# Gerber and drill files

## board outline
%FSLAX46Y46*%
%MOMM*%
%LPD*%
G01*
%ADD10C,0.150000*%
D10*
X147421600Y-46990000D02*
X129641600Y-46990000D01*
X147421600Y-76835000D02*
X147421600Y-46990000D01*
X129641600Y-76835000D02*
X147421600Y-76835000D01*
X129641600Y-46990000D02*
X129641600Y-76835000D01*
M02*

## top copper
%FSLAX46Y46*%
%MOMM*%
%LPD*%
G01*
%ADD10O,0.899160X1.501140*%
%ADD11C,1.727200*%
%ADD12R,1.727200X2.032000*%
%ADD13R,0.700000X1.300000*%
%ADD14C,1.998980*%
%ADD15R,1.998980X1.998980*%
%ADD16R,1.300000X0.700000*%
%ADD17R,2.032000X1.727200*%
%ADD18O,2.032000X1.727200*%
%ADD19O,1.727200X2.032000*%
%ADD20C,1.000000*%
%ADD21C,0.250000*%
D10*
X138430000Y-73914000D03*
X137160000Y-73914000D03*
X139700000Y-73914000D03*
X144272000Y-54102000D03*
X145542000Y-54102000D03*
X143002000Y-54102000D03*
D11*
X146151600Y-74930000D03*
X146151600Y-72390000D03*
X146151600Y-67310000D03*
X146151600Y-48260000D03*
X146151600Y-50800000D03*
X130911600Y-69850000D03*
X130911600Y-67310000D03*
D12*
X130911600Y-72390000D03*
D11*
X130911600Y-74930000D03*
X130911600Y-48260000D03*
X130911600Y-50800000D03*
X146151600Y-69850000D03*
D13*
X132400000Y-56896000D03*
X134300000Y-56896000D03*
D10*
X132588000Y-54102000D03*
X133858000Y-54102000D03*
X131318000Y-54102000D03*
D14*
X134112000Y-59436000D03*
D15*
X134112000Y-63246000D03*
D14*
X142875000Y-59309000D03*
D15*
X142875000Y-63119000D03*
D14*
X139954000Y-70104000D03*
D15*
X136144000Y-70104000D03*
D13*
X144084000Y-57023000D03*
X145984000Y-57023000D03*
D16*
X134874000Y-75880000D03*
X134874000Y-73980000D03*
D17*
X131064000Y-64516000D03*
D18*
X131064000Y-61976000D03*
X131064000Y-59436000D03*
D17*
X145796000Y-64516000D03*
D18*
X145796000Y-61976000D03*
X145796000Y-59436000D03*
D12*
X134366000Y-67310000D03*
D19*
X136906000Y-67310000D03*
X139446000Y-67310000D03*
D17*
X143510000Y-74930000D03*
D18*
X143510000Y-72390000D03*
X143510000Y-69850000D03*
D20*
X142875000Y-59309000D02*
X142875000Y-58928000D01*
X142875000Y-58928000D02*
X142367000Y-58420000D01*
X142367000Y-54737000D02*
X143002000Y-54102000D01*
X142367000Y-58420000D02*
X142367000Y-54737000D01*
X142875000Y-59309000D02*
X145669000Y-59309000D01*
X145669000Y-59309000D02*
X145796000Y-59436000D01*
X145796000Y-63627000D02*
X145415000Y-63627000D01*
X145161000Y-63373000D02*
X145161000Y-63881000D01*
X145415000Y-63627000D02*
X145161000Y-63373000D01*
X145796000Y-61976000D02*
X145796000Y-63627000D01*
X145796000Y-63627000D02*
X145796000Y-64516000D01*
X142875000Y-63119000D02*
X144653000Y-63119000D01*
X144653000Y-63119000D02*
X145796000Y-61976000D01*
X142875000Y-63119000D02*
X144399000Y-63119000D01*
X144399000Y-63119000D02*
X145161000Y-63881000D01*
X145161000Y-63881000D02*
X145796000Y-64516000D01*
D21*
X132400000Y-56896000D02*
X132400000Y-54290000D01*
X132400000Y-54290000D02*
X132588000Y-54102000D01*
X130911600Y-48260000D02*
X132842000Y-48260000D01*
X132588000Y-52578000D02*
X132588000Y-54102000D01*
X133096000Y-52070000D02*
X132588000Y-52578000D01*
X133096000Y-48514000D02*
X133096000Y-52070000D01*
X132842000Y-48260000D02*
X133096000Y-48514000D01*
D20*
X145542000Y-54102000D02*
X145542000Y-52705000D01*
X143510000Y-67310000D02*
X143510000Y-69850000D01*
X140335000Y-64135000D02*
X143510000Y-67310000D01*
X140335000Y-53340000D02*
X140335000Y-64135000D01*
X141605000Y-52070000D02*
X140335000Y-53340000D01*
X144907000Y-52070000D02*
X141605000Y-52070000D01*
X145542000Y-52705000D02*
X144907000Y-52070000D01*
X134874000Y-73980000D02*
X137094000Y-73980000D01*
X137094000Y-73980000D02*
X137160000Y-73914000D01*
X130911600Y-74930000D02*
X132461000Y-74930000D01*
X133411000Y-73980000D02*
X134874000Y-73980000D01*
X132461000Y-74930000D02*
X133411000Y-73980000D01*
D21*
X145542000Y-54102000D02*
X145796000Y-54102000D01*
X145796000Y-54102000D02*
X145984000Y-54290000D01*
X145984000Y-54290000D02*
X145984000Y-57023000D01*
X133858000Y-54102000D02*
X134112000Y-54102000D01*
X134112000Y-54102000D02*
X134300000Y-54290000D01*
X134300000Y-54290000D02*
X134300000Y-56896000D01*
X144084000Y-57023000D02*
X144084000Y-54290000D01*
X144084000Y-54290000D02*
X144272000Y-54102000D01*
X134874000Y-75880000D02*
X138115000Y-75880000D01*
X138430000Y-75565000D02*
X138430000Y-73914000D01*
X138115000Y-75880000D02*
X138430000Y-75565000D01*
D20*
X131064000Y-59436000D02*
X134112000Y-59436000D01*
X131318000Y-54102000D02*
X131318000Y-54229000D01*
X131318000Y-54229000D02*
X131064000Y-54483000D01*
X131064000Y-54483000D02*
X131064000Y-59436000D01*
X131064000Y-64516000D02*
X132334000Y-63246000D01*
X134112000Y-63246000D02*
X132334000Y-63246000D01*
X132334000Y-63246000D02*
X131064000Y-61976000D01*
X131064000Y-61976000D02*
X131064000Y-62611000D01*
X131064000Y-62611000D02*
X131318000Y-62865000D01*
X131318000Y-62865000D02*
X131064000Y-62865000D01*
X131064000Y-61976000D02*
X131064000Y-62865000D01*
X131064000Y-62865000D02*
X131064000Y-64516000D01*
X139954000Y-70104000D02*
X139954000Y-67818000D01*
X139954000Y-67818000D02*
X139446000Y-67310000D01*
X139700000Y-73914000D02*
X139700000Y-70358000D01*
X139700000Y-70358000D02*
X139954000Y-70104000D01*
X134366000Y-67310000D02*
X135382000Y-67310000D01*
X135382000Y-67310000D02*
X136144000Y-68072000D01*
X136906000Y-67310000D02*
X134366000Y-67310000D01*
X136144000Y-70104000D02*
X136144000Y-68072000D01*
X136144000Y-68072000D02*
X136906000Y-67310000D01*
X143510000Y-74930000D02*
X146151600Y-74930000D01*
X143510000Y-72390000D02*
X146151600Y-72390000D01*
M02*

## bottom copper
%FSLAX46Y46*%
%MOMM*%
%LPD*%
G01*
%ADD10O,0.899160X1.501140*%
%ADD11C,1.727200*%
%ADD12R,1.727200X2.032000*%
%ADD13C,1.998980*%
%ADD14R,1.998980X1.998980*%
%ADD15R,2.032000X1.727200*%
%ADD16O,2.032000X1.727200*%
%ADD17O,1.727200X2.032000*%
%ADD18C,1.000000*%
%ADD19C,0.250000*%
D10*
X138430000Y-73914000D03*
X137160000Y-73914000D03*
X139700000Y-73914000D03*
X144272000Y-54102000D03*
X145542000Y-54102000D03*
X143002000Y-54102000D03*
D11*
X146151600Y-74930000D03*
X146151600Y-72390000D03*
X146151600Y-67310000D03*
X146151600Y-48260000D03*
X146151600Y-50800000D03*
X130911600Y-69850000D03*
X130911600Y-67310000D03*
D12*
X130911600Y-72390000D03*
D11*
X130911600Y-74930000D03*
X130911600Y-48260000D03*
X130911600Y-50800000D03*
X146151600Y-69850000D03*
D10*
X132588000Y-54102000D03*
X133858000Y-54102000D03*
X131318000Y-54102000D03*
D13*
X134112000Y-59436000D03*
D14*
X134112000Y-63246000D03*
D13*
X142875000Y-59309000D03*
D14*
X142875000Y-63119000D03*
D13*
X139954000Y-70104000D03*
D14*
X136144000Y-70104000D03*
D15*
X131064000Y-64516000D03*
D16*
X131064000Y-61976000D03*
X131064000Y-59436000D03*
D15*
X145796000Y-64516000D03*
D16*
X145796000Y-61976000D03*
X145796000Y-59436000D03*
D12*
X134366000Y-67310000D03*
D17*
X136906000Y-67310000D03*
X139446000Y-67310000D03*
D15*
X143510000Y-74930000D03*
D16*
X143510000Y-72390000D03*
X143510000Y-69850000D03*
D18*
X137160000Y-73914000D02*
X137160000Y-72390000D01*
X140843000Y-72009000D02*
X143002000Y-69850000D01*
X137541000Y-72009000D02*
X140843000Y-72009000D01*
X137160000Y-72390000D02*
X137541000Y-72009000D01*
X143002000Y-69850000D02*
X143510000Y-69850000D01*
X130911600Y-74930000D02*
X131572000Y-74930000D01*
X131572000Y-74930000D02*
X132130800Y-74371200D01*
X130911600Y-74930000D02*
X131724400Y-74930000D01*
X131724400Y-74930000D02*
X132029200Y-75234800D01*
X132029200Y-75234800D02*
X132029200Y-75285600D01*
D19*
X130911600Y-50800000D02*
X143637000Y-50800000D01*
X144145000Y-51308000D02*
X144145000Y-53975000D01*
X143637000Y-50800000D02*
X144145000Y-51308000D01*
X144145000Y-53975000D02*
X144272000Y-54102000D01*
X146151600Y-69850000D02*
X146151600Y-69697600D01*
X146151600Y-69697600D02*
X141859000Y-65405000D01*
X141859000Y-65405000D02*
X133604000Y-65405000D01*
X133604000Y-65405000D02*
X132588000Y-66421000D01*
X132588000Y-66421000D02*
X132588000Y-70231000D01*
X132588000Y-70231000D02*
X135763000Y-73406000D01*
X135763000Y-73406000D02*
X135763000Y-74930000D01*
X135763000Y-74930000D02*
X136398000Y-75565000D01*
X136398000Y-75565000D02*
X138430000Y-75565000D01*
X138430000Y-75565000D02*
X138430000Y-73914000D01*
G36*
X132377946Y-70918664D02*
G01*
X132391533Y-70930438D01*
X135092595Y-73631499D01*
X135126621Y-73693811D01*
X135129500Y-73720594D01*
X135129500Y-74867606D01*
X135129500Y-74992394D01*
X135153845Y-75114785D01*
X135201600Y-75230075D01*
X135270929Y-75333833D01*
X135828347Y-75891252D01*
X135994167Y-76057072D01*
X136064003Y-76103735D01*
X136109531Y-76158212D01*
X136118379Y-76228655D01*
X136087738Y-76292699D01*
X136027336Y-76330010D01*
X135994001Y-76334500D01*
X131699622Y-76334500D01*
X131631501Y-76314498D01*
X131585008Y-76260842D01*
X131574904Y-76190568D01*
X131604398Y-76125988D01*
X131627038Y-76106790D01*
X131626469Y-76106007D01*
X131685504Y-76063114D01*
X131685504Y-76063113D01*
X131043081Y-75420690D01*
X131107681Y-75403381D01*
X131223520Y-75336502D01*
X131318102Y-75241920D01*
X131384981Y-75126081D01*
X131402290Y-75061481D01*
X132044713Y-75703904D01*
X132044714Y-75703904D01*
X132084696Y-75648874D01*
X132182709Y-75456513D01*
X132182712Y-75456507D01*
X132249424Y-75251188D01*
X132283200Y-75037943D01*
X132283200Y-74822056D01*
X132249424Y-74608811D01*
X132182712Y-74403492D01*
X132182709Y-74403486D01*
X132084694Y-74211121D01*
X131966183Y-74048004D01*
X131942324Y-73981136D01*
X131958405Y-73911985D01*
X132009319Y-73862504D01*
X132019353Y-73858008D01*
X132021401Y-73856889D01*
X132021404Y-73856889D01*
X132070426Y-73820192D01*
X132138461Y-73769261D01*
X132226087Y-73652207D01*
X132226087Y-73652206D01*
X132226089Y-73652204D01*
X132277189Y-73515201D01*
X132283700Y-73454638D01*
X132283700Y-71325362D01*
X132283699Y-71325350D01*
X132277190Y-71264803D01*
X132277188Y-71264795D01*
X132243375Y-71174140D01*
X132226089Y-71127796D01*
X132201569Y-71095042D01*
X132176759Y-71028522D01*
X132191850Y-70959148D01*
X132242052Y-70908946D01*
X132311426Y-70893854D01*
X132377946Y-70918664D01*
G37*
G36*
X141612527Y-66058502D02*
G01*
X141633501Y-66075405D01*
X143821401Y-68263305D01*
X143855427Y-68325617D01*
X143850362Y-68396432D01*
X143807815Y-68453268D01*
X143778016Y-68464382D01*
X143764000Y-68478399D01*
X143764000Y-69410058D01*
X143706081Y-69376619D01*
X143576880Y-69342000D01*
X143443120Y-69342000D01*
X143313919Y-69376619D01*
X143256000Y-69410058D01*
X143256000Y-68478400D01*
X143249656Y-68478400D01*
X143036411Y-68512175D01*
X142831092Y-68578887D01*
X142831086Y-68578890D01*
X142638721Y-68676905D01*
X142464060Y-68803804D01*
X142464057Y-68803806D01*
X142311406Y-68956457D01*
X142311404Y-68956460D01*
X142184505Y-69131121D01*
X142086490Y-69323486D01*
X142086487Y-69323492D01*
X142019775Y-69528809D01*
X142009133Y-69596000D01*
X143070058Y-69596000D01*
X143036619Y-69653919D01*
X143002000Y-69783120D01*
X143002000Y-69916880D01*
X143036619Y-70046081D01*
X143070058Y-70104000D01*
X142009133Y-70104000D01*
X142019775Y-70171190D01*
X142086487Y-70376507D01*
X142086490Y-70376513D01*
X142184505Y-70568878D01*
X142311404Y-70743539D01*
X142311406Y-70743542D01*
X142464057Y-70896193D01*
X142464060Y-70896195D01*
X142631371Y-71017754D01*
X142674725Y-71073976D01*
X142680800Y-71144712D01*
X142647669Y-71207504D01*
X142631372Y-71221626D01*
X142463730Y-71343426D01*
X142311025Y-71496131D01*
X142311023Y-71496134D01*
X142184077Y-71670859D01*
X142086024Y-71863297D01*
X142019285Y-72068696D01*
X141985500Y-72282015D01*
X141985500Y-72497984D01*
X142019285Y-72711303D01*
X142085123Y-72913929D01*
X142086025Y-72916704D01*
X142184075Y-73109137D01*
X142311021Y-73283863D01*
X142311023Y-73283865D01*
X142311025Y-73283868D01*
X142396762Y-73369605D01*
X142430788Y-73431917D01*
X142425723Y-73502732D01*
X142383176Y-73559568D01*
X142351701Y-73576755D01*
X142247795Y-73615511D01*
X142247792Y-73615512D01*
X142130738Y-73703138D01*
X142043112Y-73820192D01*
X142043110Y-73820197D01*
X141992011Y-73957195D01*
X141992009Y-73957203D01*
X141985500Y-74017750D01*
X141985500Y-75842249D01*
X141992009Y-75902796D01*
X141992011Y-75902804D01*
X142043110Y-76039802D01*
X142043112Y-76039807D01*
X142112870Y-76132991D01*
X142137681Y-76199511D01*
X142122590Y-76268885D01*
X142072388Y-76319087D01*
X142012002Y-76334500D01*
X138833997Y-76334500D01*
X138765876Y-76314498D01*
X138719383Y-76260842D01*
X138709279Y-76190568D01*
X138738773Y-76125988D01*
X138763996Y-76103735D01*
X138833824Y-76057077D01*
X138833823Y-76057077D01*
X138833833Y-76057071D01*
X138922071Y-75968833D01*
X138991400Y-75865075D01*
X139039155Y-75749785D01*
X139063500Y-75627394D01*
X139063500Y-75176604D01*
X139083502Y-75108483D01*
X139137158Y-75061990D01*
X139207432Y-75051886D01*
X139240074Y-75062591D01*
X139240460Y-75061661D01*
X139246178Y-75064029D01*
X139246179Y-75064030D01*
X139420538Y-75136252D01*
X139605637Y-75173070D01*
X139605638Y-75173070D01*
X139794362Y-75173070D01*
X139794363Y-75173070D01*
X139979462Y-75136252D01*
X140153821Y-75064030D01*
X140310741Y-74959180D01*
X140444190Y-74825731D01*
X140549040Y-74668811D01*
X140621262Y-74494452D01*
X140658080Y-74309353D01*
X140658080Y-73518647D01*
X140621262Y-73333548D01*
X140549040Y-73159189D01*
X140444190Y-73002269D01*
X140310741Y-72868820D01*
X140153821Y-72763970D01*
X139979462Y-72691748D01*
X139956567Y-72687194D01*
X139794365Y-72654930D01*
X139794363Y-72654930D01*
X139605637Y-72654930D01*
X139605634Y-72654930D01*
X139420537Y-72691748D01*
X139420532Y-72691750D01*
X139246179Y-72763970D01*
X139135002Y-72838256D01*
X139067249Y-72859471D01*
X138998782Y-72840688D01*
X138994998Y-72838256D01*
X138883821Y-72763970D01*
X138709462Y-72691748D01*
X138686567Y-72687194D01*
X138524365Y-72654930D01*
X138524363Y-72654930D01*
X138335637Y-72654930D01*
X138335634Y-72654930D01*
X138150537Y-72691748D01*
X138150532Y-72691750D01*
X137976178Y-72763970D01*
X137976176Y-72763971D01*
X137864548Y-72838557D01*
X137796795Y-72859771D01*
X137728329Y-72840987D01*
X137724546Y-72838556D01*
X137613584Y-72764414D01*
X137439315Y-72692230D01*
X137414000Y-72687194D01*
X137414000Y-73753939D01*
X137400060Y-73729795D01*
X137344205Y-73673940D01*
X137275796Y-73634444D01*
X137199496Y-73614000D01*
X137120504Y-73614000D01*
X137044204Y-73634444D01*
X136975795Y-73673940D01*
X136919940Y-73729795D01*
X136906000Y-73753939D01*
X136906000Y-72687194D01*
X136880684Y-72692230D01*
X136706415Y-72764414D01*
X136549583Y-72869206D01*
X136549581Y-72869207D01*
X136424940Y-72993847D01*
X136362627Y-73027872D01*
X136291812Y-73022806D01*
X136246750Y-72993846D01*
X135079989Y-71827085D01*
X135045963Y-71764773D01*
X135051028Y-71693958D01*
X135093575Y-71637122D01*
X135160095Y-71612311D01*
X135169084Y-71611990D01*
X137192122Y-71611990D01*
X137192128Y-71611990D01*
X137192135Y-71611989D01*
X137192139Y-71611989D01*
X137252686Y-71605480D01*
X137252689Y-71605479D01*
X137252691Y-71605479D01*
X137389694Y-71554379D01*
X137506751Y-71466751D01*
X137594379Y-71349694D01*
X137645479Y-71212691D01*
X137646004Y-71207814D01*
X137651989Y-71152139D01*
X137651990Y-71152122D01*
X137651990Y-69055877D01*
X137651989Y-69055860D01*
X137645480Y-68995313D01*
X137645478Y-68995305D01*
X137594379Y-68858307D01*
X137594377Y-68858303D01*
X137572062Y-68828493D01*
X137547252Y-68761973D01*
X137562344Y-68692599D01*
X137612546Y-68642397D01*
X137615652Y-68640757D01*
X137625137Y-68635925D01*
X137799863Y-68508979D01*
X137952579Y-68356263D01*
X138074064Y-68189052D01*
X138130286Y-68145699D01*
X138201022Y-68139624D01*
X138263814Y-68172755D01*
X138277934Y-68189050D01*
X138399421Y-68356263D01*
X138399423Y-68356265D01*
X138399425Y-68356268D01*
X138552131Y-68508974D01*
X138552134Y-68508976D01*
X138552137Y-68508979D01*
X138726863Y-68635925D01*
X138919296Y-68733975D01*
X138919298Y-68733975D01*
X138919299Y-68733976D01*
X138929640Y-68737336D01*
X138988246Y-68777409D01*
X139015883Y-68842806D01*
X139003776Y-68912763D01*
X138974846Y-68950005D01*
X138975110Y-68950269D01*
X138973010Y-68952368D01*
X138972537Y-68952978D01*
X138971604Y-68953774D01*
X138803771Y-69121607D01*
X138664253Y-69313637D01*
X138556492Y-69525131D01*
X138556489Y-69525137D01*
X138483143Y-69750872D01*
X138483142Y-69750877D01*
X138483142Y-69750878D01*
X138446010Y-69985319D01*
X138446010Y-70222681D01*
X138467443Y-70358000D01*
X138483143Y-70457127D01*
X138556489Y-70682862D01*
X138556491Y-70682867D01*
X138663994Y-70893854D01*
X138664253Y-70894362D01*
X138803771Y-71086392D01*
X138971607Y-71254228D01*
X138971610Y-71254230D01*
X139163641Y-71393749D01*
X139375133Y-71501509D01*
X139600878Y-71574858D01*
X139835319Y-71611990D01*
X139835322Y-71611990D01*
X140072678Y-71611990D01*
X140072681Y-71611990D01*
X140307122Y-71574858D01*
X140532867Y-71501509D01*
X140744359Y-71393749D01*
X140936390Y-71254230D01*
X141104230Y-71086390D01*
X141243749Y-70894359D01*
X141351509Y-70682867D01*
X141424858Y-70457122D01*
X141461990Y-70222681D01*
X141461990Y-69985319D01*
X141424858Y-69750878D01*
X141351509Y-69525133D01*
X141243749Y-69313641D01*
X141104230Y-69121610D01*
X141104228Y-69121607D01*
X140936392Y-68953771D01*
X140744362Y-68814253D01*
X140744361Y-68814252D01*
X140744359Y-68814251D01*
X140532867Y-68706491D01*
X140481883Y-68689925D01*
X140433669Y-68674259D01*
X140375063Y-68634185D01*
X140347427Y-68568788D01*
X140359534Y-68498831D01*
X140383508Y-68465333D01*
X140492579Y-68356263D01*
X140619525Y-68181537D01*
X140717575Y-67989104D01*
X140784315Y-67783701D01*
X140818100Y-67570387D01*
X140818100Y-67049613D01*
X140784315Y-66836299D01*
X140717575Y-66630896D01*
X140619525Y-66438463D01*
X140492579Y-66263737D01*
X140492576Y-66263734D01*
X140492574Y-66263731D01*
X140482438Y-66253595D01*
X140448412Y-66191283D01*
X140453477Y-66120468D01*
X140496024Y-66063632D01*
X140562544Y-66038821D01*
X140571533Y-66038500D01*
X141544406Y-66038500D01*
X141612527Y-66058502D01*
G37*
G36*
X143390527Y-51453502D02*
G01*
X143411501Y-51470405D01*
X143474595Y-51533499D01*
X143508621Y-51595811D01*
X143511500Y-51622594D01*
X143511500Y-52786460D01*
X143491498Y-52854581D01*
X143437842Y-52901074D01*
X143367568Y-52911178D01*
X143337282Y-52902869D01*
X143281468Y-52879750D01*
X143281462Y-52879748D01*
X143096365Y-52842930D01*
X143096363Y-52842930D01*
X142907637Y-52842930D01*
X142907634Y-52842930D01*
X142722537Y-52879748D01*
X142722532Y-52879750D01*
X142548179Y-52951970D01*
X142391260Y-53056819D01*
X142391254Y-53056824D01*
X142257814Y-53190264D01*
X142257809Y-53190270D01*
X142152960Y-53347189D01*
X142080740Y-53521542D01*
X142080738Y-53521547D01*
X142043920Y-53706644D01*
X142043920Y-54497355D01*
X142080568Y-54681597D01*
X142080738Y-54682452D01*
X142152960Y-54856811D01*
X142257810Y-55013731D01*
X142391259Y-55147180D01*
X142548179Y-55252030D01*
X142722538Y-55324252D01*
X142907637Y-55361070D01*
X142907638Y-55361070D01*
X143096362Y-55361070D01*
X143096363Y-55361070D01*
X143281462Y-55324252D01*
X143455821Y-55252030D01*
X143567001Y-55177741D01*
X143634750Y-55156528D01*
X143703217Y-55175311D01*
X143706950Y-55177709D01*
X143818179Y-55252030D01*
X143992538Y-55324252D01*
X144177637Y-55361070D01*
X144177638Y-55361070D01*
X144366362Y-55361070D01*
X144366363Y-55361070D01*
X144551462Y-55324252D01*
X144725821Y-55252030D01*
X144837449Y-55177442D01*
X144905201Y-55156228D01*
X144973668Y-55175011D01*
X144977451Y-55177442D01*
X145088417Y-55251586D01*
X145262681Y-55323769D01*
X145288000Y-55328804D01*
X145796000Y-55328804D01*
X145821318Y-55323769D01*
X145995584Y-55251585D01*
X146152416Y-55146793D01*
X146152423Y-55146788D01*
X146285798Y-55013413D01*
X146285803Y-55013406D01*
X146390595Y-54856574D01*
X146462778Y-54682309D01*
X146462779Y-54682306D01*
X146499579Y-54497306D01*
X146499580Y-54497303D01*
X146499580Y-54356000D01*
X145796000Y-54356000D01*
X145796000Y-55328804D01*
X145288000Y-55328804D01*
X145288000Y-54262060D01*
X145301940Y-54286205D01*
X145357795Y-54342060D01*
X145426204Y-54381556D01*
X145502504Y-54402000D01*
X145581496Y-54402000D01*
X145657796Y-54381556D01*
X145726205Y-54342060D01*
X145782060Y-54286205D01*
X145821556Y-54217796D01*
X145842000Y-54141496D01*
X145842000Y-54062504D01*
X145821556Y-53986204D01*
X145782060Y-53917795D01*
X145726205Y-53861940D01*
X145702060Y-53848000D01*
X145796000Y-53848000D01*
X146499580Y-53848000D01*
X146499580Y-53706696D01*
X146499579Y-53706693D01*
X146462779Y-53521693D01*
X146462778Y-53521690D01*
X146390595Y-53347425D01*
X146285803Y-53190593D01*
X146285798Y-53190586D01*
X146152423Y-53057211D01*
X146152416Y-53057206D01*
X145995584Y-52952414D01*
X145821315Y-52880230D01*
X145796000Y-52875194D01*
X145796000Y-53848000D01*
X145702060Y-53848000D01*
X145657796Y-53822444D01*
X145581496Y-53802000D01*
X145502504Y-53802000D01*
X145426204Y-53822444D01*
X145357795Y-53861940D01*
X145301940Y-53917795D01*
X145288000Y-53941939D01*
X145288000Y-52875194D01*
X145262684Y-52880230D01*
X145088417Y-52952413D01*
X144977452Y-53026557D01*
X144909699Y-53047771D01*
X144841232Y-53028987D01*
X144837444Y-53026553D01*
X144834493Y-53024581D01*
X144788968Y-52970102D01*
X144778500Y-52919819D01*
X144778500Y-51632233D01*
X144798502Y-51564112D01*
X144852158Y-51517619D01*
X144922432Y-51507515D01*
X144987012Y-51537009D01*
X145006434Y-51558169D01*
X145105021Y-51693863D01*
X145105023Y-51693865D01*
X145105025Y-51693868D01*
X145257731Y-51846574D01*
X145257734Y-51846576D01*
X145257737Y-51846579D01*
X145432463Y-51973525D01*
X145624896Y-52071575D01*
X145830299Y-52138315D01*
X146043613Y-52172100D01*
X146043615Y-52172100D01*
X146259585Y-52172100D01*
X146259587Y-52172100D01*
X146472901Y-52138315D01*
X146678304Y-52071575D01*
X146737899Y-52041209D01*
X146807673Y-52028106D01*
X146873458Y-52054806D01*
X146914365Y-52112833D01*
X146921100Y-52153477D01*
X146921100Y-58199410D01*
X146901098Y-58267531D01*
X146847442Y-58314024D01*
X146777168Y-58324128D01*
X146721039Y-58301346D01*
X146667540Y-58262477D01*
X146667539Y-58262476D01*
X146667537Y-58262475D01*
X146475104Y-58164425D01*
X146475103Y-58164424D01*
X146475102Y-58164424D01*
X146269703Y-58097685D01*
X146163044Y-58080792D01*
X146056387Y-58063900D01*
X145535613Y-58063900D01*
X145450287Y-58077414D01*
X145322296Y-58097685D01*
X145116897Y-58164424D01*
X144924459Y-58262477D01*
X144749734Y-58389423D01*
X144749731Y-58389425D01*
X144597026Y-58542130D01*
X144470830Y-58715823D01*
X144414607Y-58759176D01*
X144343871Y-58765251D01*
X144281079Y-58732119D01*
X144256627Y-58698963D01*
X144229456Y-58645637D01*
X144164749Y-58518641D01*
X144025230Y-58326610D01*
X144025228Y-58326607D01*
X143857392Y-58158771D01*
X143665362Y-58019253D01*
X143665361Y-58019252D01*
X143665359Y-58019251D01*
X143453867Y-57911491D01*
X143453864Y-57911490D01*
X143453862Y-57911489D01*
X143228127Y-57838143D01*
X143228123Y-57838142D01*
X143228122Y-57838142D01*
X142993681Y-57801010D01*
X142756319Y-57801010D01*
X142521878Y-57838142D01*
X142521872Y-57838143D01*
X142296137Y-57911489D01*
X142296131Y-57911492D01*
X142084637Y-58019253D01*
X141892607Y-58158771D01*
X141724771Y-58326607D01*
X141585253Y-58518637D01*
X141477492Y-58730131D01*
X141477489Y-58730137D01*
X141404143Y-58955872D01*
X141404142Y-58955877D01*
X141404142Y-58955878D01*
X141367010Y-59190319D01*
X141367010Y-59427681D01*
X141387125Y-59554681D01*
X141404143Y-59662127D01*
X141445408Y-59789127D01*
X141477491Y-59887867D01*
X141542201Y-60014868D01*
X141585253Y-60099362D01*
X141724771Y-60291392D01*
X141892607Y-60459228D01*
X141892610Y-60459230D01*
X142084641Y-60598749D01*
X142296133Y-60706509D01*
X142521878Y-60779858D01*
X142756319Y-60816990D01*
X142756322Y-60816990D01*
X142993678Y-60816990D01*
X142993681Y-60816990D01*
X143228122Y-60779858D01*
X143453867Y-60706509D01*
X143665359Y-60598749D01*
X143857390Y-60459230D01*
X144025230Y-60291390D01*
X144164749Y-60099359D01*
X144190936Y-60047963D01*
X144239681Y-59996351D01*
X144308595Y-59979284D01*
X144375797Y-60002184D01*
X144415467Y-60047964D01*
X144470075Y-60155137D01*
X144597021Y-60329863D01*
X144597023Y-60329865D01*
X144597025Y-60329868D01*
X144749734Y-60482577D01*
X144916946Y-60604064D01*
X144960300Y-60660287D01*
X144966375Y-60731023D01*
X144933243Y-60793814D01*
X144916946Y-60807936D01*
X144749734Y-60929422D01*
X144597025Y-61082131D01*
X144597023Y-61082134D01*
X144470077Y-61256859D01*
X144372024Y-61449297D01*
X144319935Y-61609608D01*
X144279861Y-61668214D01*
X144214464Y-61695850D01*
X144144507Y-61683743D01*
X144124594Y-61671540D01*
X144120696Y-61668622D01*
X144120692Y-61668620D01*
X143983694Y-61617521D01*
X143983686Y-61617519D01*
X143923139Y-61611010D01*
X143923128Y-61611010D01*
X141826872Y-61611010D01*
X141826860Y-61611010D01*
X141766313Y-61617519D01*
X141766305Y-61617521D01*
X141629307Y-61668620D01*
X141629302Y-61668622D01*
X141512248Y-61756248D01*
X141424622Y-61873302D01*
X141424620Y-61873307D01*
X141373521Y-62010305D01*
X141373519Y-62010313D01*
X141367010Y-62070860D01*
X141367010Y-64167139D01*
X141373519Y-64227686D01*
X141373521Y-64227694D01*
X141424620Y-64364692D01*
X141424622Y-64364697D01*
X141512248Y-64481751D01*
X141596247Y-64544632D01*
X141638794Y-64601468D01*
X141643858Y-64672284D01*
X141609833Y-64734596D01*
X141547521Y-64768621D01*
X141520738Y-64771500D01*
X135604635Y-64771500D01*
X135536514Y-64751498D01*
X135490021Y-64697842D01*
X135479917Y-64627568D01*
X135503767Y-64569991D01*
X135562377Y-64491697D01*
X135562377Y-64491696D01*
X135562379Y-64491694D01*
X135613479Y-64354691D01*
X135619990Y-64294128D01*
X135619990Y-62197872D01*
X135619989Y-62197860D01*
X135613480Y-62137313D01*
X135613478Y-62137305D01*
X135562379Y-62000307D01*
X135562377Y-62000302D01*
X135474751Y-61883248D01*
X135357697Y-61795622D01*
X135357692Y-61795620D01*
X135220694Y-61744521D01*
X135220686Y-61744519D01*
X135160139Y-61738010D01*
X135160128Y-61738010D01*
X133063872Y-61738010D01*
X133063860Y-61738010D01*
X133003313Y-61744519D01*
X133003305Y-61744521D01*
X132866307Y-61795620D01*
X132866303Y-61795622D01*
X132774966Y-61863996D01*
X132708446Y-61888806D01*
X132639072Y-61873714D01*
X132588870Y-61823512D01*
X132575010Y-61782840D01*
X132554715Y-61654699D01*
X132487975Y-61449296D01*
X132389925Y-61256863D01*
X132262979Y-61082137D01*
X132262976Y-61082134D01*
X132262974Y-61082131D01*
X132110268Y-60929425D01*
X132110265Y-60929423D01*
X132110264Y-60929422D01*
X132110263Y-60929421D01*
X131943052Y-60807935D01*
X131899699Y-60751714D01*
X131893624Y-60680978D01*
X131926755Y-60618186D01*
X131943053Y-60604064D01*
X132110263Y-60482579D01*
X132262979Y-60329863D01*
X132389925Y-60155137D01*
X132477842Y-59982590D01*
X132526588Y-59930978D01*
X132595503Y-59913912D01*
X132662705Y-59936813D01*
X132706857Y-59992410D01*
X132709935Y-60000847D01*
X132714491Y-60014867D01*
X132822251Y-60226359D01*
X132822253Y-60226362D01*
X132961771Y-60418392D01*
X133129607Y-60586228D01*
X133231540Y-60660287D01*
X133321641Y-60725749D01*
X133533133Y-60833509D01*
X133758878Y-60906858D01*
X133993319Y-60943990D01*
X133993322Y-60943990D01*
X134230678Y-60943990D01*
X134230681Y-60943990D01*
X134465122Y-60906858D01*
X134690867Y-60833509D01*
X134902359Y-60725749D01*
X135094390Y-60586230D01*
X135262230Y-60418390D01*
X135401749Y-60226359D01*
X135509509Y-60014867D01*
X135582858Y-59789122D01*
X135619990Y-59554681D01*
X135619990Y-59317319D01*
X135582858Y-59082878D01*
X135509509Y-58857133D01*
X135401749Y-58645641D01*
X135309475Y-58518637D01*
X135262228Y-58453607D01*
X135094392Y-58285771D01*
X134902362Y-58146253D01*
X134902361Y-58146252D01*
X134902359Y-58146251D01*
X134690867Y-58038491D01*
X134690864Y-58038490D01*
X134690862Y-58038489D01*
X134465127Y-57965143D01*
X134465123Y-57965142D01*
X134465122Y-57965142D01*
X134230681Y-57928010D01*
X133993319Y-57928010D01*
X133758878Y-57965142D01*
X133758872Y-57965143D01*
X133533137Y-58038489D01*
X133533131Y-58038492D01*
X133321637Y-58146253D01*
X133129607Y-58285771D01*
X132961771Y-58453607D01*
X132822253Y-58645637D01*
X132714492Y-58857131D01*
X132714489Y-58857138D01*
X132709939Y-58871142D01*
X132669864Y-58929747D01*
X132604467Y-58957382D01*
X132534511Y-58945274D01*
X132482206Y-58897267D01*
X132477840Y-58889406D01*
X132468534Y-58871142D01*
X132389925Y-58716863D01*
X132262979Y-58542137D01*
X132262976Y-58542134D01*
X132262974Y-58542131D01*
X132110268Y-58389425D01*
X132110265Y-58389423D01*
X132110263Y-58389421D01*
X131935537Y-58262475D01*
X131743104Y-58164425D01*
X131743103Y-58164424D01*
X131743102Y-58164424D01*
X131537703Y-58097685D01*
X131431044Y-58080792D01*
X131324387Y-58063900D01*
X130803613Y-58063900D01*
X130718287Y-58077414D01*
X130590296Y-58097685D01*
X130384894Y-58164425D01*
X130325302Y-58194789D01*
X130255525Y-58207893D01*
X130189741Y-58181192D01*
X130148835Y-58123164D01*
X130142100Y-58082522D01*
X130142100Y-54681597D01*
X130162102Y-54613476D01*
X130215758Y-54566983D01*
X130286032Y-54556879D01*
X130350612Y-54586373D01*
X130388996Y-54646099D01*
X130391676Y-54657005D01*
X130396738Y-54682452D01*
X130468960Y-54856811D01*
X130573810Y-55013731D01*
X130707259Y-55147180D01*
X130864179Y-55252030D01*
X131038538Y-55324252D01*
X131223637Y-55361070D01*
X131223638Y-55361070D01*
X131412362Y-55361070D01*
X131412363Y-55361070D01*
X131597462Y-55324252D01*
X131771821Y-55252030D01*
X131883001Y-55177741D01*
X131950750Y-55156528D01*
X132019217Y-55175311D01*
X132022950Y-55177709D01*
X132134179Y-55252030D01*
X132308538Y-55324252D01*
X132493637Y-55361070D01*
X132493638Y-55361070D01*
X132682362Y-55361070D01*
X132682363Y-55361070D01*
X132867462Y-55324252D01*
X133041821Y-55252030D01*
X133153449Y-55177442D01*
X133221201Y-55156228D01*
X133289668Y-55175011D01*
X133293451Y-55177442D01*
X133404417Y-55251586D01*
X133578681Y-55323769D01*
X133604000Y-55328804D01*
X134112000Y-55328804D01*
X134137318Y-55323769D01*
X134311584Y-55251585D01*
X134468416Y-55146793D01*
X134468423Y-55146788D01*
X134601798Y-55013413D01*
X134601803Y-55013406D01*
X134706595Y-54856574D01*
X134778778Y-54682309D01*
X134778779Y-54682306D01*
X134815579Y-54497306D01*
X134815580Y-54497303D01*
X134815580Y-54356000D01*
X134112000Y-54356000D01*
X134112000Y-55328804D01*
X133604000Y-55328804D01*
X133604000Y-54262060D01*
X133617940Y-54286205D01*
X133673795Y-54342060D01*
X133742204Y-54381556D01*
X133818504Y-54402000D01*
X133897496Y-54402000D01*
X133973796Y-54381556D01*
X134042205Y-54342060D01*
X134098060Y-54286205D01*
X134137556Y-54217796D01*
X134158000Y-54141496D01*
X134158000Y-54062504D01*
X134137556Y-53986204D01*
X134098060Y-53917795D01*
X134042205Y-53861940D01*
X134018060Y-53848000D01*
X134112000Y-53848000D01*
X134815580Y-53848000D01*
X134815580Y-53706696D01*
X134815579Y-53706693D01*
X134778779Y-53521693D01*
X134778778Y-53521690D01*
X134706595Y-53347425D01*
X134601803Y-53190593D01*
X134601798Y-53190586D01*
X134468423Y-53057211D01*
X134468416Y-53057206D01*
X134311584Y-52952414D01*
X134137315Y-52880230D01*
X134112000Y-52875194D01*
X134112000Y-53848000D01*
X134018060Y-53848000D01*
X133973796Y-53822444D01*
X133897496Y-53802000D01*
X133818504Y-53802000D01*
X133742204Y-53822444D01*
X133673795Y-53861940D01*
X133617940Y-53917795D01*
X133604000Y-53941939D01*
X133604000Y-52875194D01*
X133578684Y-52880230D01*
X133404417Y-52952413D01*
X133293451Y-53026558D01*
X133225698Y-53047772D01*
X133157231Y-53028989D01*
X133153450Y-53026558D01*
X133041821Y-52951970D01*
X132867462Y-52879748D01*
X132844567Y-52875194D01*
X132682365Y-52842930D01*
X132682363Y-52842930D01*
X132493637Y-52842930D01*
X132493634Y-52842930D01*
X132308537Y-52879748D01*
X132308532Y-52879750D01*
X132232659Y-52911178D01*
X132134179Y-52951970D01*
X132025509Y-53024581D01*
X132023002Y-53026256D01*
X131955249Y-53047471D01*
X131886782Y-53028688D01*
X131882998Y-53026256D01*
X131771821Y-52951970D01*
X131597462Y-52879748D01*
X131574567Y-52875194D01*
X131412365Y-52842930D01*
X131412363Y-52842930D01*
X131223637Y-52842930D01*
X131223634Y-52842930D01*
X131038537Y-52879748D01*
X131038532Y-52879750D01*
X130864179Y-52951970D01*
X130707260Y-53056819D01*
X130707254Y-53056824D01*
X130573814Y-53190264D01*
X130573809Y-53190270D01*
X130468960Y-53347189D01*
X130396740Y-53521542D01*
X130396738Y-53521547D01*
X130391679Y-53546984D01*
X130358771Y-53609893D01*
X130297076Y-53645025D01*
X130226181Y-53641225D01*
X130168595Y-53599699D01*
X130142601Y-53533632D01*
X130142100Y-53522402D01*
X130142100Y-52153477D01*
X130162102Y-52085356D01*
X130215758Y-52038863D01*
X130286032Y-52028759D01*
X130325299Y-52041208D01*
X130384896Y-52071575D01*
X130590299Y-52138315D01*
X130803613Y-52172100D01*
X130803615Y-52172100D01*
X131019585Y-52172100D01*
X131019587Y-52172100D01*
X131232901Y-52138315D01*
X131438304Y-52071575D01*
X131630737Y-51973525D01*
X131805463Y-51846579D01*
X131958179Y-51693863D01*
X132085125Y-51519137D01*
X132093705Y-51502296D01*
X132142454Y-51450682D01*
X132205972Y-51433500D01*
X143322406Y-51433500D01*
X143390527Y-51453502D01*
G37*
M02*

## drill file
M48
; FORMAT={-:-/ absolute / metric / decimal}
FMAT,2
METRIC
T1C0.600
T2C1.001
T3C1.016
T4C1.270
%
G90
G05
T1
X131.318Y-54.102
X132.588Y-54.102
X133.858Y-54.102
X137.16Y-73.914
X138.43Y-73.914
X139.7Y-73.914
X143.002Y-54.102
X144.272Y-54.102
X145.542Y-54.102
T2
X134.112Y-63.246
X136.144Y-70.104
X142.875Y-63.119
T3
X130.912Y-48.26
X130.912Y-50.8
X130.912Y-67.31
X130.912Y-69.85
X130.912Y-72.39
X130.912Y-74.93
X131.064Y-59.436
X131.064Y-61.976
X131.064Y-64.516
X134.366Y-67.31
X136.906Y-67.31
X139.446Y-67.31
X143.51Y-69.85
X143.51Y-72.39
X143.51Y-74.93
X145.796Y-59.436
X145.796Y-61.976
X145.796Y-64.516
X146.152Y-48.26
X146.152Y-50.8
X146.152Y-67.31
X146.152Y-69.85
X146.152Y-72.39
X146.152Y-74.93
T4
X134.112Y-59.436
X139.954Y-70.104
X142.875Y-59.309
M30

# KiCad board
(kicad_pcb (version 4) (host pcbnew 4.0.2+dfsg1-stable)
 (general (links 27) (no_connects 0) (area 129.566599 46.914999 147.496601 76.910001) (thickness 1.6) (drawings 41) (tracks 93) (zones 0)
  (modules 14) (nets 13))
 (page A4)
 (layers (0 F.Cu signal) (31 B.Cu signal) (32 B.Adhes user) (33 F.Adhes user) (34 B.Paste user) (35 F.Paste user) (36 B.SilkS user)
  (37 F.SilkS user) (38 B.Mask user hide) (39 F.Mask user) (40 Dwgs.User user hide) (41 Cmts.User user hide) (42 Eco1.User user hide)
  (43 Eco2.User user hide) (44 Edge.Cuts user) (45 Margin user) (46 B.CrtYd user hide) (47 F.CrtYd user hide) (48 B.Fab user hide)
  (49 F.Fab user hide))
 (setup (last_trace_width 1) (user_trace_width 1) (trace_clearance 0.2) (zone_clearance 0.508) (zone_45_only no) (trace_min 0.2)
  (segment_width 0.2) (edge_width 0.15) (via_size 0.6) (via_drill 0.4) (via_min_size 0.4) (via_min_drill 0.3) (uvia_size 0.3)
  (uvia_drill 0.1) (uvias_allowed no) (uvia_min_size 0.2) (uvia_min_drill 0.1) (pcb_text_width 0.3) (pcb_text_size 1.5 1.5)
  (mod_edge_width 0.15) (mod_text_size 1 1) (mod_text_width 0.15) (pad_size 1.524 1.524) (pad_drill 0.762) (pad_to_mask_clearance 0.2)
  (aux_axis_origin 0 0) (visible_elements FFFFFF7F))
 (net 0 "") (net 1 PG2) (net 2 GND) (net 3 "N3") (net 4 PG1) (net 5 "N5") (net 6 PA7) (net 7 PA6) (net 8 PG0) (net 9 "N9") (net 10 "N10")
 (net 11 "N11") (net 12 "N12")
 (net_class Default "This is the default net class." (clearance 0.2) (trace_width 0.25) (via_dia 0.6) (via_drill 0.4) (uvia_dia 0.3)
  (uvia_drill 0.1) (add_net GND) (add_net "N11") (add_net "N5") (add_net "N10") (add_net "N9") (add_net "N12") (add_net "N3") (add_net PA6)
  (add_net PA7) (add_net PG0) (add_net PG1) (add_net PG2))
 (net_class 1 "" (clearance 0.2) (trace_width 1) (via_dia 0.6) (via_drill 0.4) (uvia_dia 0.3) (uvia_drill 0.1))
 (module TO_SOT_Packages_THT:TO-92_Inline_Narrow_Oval (layer F.Cu) (at 139.7 73.914 180)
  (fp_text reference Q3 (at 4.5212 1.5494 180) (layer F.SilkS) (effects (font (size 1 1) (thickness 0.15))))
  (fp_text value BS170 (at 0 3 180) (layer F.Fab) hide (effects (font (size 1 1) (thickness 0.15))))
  (pad 2 thru_hole oval (at 1.27 0) (size 0.89916 1.50114) (drill 0.6) (layers *.Cu *.Mask F.SilkS) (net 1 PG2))
  (pad 3 thru_hole oval (at 2.54 0) (size 0.89916 1.50114) (drill 0.6) (layers *.Cu *.Mask F.SilkS) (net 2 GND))
  (pad 1 thru_hole oval (at 0 0) (size 0.89916 1.50114) (drill 0.6) (layers *.Cu *.Mask F.SilkS) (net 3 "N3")))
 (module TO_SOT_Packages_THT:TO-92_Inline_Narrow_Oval (layer F.Cu) (at 143.002 54.102)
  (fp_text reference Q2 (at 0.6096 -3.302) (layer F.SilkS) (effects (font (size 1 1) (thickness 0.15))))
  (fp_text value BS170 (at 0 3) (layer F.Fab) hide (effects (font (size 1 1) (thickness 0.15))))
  (pad 2 thru_hole oval (at 1.27 0 180) (size 0.89916 1.50114) (drill 0.6) (layers *.Cu *.Mask F.SilkS) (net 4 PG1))
  (pad 3 thru_hole oval (at 2.54 0 180) (size 0.89916 1.50114) (drill 0.6) (layers *.Cu *.Mask F.SilkS) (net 2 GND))
  (pad 1 thru_hole oval (at 0 0 180) (size 0.89916 1.50114) (drill 0.6) (layers *.Cu *.Mask F.SilkS) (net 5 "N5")))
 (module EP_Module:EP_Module (layer F.Cu) (at 133.4516 48.26)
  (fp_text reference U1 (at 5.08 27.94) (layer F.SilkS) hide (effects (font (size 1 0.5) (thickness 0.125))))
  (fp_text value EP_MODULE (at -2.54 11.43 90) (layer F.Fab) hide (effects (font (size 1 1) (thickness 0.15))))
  (pad 12 thru_hole circle (at 12.7 26.67) (size 1.7272 1.7272) (drill 1.016) (layers *.Cu *.Mask F.SilkS) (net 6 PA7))
  (pad 11 thru_hole circle (at 12.7 24.13) (size 1.7272 1.7272) (drill 1.016) (layers *.Cu *.Mask F.SilkS) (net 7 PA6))
  (pad 10 thru_hole circle (at 12.7 19.05) (size 1.7272 1.7272) (drill 1.016) (layers *.Cu *.Mask F.SilkS))
  (pad 9 thru_hole circle (at 12.7 0) (size 1.7272 1.7272) (drill 1.016) (layers *.Cu *.Mask F.SilkS))
  (pad 8 thru_hole circle (at 12.7 2.54) (size 1.7272 1.7272) (drill 1.016) (layers *.Cu *.Mask F.SilkS))
  (pad 7 thru_hole circle (at -2.54 21.59) (size 1.7272 1.7272) (drill 1.016) (layers *.Cu *.Mask F.SilkS))
  (pad 6 thru_hole circle (at -2.54 19.05) (size 1.7272 1.7272) (drill 1.016) (layers *.Cu *.Mask F.SilkS))
  (pad 1 thru_hole rect (at -2.54 24.13) (size 1.7272 2.032) (drill 1.016) (layers *.Cu *.Mask F.SilkS))
  (pad 2 thru_hole circle (at -2.54 26.67) (size 1.7272 1.7272) (drill 1.016) (layers *.Cu *.Mask F.SilkS) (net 2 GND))
  (pad 3 thru_hole circle (at -2.54 0) (size 1.7272 1.7272) (drill 1.016) (layers *.Cu *.Mask F.SilkS) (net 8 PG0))
  (pad 4 thru_hole circle (at -2.54 2.54) (size 1.7272 1.7272) (drill 1.016) (layers *.Cu *.Mask F.SilkS) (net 4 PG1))
  (pad 5 thru_hole circle (at 12.7 21.59) (size 1.7272 1.7272) (drill 1.016) (layers *.Cu *.Mask F.SilkS) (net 1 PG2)))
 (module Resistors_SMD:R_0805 (layer F.Cu) (at 133.35 56.896)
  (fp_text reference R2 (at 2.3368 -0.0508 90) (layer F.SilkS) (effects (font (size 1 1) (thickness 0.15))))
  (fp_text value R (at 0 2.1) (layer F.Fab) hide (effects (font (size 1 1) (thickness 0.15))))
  (pad 1 smd rect (at -0.95 0) (size 0.7 1.3) (layers F.Cu F.Paste F.Mask) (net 8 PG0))
  (pad 2 smd rect (at 0.95 0) (size 0.7 1.3) (layers F.Cu F.Paste F.Mask) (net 2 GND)))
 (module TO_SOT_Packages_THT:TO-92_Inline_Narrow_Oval (layer F.Cu) (at 131.318 54.102)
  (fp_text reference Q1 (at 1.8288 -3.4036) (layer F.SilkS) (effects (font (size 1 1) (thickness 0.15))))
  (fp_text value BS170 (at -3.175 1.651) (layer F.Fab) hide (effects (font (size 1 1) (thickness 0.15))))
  (pad 2 thru_hole oval (at 1.27 0 180) (size 0.89916 1.50114) (drill 0.6) (layers *.Cu *.Mask F.SilkS) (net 8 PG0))
  (pad 3 thru_hole oval (at 2.54 0 180) (size 0.89916 1.50114) (drill 0.6) (layers *.Cu *.Mask F.SilkS) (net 2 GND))
  (pad 1 thru_hole oval (at 0 0 180) (size 0.89916 1.50114) (drill 0.6) (layers *.Cu *.Mask F.SilkS) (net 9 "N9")))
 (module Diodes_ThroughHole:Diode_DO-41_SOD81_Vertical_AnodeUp (layer F.Cu) (at 134.112 63.246 90)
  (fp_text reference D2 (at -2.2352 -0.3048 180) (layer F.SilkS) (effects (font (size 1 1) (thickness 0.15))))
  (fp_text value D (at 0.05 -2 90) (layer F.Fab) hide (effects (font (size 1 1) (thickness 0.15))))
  (pad 2 thru_hole circle (at 3.81 0 90) (size 1.99898 1.99898) (drill 1.27) (layers *.Cu *.Mask F.SilkS) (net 9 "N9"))
  (pad 1 thru_hole rect (at 0 0 90) (size 1.99898 1.99898) (drill 1.00076) (layers *.Cu *.Mask F.SilkS) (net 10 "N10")))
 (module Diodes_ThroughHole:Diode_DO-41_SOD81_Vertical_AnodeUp (layer F.Cu) (at 142.875 63.119 90)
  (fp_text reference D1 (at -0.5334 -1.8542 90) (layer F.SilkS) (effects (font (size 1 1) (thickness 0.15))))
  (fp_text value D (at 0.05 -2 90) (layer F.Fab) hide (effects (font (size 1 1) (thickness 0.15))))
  (pad 2 thru_hole circle (at 3.81 0 90) (size 1.99898 1.99898) (drill 1.27) (layers *.Cu *.Mask F.SilkS) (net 5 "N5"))
  (pad 1 thru_hole rect (at 0 0 90) (size 1.99898 1.99898) (drill 1.00076) (layers *.Cu *.Mask F.SilkS) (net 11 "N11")))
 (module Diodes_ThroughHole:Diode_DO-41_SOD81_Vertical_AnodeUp (layer F.Cu) (at 136.144 70.104)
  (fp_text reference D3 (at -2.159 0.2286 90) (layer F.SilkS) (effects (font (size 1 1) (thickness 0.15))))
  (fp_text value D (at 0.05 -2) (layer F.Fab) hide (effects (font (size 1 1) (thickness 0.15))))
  (pad 2 thru_hole circle (at 3.81 0) (size 1.99898 1.99898) (drill 1.27) (layers *.Cu *.Mask F.SilkS) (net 3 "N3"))
  (pad 1 thru_hole rect (at 0 0) (size 1.99898 1.99898) (drill 1.00076) (layers *.Cu *.Mask F.SilkS) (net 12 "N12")))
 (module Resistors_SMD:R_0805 (layer F.Cu) (at 145.034 57.023)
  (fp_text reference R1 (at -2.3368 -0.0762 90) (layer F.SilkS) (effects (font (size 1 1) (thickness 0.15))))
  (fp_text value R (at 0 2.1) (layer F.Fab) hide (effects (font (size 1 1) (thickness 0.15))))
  (pad 1 smd rect (at -0.95 0) (size 0.7 1.3) (layers F.Cu F.Paste F.Mask) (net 4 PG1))
  (pad 2 smd rect (at 0.95 0) (size 0.7 1.3) (layers F.Cu F.Paste F.Mask) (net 2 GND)))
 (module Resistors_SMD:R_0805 (layer F.Cu) (at 134.874 74.93 90)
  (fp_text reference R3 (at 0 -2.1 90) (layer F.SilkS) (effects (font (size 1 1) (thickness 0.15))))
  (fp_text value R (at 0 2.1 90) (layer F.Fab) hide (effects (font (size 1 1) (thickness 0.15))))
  (pad 1 smd rect (at -0.95 0 90) (size 0.7 1.3) (layers F.Cu F.Paste F.Mask) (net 1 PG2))
  (pad 2 smd rect (at 0.95 0 90) (size 0.7 1.3) (layers F.Cu F.Paste F.Mask) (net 2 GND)))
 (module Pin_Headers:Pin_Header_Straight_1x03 (layer F.Cu) (at 131.064 64.516 180)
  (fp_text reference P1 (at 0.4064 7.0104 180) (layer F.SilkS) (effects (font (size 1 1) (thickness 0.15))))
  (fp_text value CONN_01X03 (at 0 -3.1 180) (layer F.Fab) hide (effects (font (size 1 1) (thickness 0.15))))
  (pad 1 thru_hole rect (at 0 0 180) (size 2.032 1.7272) (drill 1.016) (layers *.Cu *.Mask F.SilkS) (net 10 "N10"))
  (pad 2 thru_hole oval (at 0 2.54 180) (size 2.032 1.7272) (drill 1.016) (layers *.Cu *.Mask F.SilkS) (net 10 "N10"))
  (pad 3 thru_hole oval (at 0 5.08 180) (size 2.032 1.7272) (drill 1.016) (layers *.Cu *.Mask F.SilkS) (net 9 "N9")))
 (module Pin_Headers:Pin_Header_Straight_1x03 (layer F.Cu) (at 145.796 64.516 180)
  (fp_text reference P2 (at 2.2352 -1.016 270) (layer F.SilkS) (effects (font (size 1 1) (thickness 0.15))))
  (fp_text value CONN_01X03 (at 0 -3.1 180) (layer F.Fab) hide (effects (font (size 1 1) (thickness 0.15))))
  (pad 1 thru_hole rect (at 0 0 180) (size 2.032 1.7272) (drill 1.016) (layers *.Cu *.Mask F.SilkS) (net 11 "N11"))
  (pad 2 thru_hole oval (at 0 2.54 180) (size 2.032 1.7272) (drill 1.016) (layers *.Cu *.Mask F.SilkS) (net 11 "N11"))
  (pad 3 thru_hole oval (at 0 5.08 180) (size 2.032 1.7272) (drill 1.016) (layers *.Cu *.Mask F.SilkS) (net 5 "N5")))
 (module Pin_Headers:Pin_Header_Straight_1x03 (layer F.Cu) (at 134.366 67.31 90)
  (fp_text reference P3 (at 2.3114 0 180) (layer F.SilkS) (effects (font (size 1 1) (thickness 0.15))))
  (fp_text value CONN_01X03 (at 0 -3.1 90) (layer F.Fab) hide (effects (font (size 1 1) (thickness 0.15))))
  (pad 1 thru_hole rect (at 0 0 90) (size 2.032 1.7272) (drill 1.016) (layers *.Cu *.Mask F.SilkS) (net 12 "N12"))
  (pad 2 thru_hole oval (at 0 2.54 90) (size 2.032 1.7272) (drill 1.016) (layers *.Cu *.Mask F.SilkS) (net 12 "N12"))
  (pad 3 thru_hole oval (at 0 5.08 90) (size 2.032 1.7272) (drill 1.016) (layers *.Cu *.Mask F.SilkS) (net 3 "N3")))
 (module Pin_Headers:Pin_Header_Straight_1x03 (layer F.Cu) (at 143.51 74.93 180)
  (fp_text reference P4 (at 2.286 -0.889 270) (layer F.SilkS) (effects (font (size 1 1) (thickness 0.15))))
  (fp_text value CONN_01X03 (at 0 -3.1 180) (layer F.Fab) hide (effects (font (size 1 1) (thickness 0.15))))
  (pad 1 thru_hole rect (at 0 0 180) (size 2.032 1.7272) (drill 1.016) (layers *.Cu *.Mask F.SilkS) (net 6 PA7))
  (pad 2 thru_hole oval (at 0 2.54 180) (size 2.032 1.7272) (drill 1.016) (layers *.Cu *.Mask F.SilkS) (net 7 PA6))
  (pad 3 thru_hole oval (at 0 5.08 180) (size 2.032 1.7272) (drill 1.016) (layers *.Cu *.Mask F.SilkS) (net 2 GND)))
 (gr_line (start 147.4216 46.99) (end 129.6416 46.99) (angle 90) (layer Edge.Cuts) (width 0.15))
 (gr_line (start 147.4216 76.835) (end 147.4216 46.99) (angle 90) (layer Edge.Cuts) (width 0.15))
 (gr_line (start 129.6416 76.835) (end 147.4216 76.835) (angle 90) (layer Edge.Cuts) (width 0.15))
 (gr_line (start 129.6416 46.99) (end 129.6416 76.835) (angle 90) (layer Edge.Cuts) (width 0.15))
 (segment (start 142.875 59.309) (end 142.875 58.928) (width 1) (layer F.Cu) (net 5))
 (segment (start 142.875 58.928) (end 142.367 58.42) (width 1) (layer F.Cu) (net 5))
 (segment (start 142.367 54.737) (end 143.002 54.102) (width 1) (layer F.Cu) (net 5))
 (segment (start 142.367 58.42) (end 142.367 54.737) (width 1) (layer F.Cu) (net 5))
 (segment (start 142.875 59.309) (end 145.669 59.309) (width 1) (layer F.Cu) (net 5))
 (segment (start 145.669 59.309) (end 145.796 59.436) (width 1) (layer F.Cu) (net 5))
 (segment (start 145.796 63.627) (end 145.415 63.627) (width 1) (layer F.Cu) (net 11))
 (segment (start 145.161 63.373) (end 145.161 63.881) (width 1) (layer F.Cu) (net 11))
 (segment (start 145.415 63.627) (end 145.161 63.373) (width 1) (layer F.Cu) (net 11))
 (segment (start 145.796 61.976) (end 145.796 63.627) (width 1) (layer F.Cu) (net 11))
 (segment (start 145.796 63.627) (end 145.796 64.516) (width 1) (layer F.Cu) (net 11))
 (segment (start 142.875 63.119) (end 144.653 63.119) (width 1) (layer F.Cu) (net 11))
 (segment (start 144.653 63.119) (end 145.796 61.976) (width 1) (layer F.Cu) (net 11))
 (segment (start 142.875 63.119) (end 144.399 63.119) (width 1) (layer F.Cu) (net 11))
 (segment (start 144.399 63.119) (end 145.161 63.881) (width 1) (layer F.Cu) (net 11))
 (segment (start 145.161 63.881) (end 145.796 64.516) (width 1) (layer F.Cu) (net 11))
 (segment (start 132.4 56.896) (end 132.4 54.29) (width 0.25) (layer F.Cu) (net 8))
 (segment (start 132.4 54.29) (end 132.588 54.102) (width 0.25) (layer F.Cu) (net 8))
 (segment (start 130.9116 48.26) (end 132.842 48.26) (width 0.25) (layer F.Cu) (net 8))
 (segment (start 132.588 52.578) (end 132.588 54.102) (width 0.25) (layer F.Cu) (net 8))
 (segment (start 133.096 52.07) (end 132.588 52.578) (width 0.25) (layer F.Cu) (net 8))
 (segment (start 133.096 48.514) (end 133.096 52.07) (width 0.25) (layer F.Cu) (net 8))
 (segment (start 132.842 48.26) (end 133.096 48.514) (width 0.25) (layer F.Cu) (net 8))
 (segment (start 145.542 54.102) (end 145.542 52.705) (width 1) (layer F.Cu) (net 2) (status 400000))
 (segment (start 143.51 67.31) (end 143.51 69.85) (width 1) (layer F.Cu) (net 2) (status 800000))
 (segment (start 140.335 64.135) (end 143.51 67.31) (width 1) (layer F.Cu) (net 2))
 (segment (start 140.335 53.34) (end 140.335 64.135) (width 1) (layer F.Cu) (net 2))
 (segment (start 141.605 52.07) (end 140.335 53.34) (width 1) (layer F.Cu) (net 2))
 (segment (start 144.907 52.07) (end 141.605 52.07) (width 1) (layer F.Cu) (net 2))
 (segment (start 145.542 52.705) (end 144.907 52.07) (width 1) (layer F.Cu) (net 2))
 (segment (start 137.16 73.914) (end 137.16 72.39) (width 1) (layer B.Cu) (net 2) (status 400000))
 (segment (start 140.843 72.009) (end 143.002 69.85) (width 1) (layer B.Cu) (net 2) (status 800000))
 (segment (start 137.541 72.009) (end 140.843 72.009) (width 1) (layer B.Cu) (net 2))
 (segment (start 137.16 72.39) (end 137.541 72.009) (width 1) (layer B.Cu) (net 2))
 (segment (start 143.002 69.85) (end 143.51 69.85) (width 1) (layer B.Cu) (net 2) (status C00000))
 (segment (start 134.874 73.98) (end 137.094 73.98) (width 1) (layer F.Cu) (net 2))
 (segment (start 137.094 73.98) (end 137.16 73.914) (width 1) (layer F.Cu) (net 2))
 (segment (start 130.9116 74.93) (end 132.461 74.93) (width 1) (layer F.Cu) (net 2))
 (segment (start 133.411 73.98) (end 134.874 73.98) (width 1) (layer F.Cu) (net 2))
 (segment (start 132.461 74.93) (end 133.411 73.98) (width 1) (layer F.Cu) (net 2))
 (segment (start 130.9116 74.93) (end 131.572 74.93) (width 1) (layer B.Cu) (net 2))
 (segment (start 131.572 74.93) (end 132.1308 74.3712) (width 1) (layer B.Cu) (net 2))
 (segment (start 130.9116 74.93) (end 131.7244 74.93) (width 1) (layer B.Cu) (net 2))
 (segment (start 131.7244 74.93) (end 132.0292 75.2348) (width 1) (layer B.Cu) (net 2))
 (segment (start 132.0292 75.2348) (end 132.0292 75.2856) (width 1) (layer B.Cu) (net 2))
 (segment (start 145.542 54.102) (end 145.796 54.102) (width 0.25) (layer F.Cu) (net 2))
 (segment (start 145.796 54.102) (end 145.984 54.29) (width 0.25) (layer F.Cu) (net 2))
 (segment (start 145.984 54.29) (end 145.984 57.023) (width 0.25) (layer F.Cu) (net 2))
 (segment (start 133.858 54.102) (end 134.112 54.102) (width 0.25) (layer F.Cu) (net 2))
 (segment (start 134.112 54.102) (end 134.3 54.29) (width 0.25) (layer F.Cu) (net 2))
 (segment (start 134.3 54.29) (end 134.3 56.896) (width 0.25) (layer F.Cu) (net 2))
 (segment (start 144.084 57.023) (end 144.084 54.29) (width 0.25) (layer F.Cu) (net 4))
 (segment (start 144.084 54.29) (end 144.272 54.102) (width 0.25) (layer F.Cu) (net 4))
 (segment (start 130.9116 50.8) (end 143.637 50.8) (width 0.25) (layer B.Cu) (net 4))
 (segment (start 144.145 51.308) (end 144.145 53.975) (width 0.25) (layer B.Cu) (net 4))
 (segment (start 143.637 50.8) (end 144.145 51.308) (width 0.25) (layer B.Cu) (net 4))
 (segment (start 144.145 53.975) (end 144.272 54.102) (width 0.25) (layer B.Cu) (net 4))
 (segment (start 146.1516 69.85) (end 146.1516 69.6976) (width 0.25) (layer B.Cu) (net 1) (status C00000))
 (segment (start 146.1516 69.6976) (end 141.859 65.405) (width 0.25) (layer B.Cu) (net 1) (status 400000))
 (segment (start 141.859 65.405) (end 133.604 65.405) (width 0.25) (layer B.Cu) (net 1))
 (segment (start 133.604 65.405) (end 132.588 66.421) (width 0.25) (layer B.Cu) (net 1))
 (segment (start 132.588 66.421) (end 132.588 70.231) (width 0.25) (layer B.Cu) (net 1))
 (segment (start 132.588 70.231) (end 135.763 73.406) (width 0.25) (layer B.Cu) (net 1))
 (segment (start 135.763 73.406) (end 135.763 74.93) (width 0.25) (layer B.Cu) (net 1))
 (segment (start 135.763 74.93) (end 136.398 75.565) (width 0.25) (layer B.Cu) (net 1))
 (segment (start 136.398 75.565) (end 138.43 75.565) (width 0.25) (layer B.Cu) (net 1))
 (segment (start 138.43 75.565) (end 138.43 73.914) (width 0.25) (layer B.Cu) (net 1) (status 800000))
 (segment (start 134.874 75.88) (end 138.115 75.88) (width 0.25) (layer F.Cu) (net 1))
 (segment (start 138.43 75.565) (end 138.43 73.914) (width 0.25) (layer F.Cu) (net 1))
 (segment (start 138.115 75.88) (end 138.43 75.565) (width 0.25) (layer F.Cu) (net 1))
 (segment (start 131.064 59.436) (end 134.112 59.436) (width 1) (layer F.Cu) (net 9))
 (segment (start 131.318 54.102) (end 131.318 54.229) (width 1) (layer F.Cu) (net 9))
 (segment (start 131.318 54.229) (end 131.064 54.483) (width 1) (layer F.Cu) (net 9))
 (segment (start 131.064 54.483) (end 131.064 59.436) (width 1) (layer F.Cu) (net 9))
 (segment (start 131.064 64.516) (end 132.334 63.246) (width 1) (layer F.Cu) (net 10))
 (segment (start 134.112 63.246) (end 132.334 63.246) (width 1) (layer F.Cu) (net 10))
 (segment (start 132.334 63.246) (end 131.064 61.976) (width 1) (layer F.Cu) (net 10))
 (segment (start 131.064 61.976) (end 131.064 62.611) (width 1) (layer F.Cu) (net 10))
 (segment (start 131.064 62.611) (end 131.318 62.865) (width 1) (layer F.Cu) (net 10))
 (segment (start 131.318 62.865) (end 131.064 62.865) (width 1) (layer F.Cu) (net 10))
 (segment (start 131.064 61.976) (end 131.064 62.865) (width 1) (layer F.Cu) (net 10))
 (segment (start 131.064 62.865) (end 131.064 64.516) (width 1) (layer F.Cu) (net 10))
 (segment (start 139.954 70.104) (end 139.954 67.818) (width 1) (layer F.Cu) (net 3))
 (segment (start 139.954 67.818) (end 139.446 67.31) (width 1) (layer F.Cu) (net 3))
 (segment (start 139.7 73.914) (end 139.7 70.358) (width 1) (layer F.Cu) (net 3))
 (segment (start 139.7 70.358) (end 139.954 70.104) (width 1) (layer F.Cu) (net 3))
 (segment (start 134.366 67.31) (end 135.382 67.31) (width 1) (layer F.Cu) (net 12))
 (segment (start 135.382 67.31) (end 136.144 68.072) (width 1) (layer F.Cu) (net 12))
 (segment (start 136.906 67.31) (end 134.366 67.31) (width 1) (layer F.Cu) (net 12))
 (segment (start 136.144 70.104) (end 136.144 68.072) (width 1) (layer F.Cu) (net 12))
 (segment (start 136.144 68.072) (end 136.906 67.31) (width 1) (layer F.Cu) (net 12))
 (segment (start 143.51 74.93) (end 146.1516 74.93) (width 1) (layer F.Cu) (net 6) (status C00000))
 (segment (start 143.51 72.39) (end 146.1516 72.39) (width 1) (layer F.Cu) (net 7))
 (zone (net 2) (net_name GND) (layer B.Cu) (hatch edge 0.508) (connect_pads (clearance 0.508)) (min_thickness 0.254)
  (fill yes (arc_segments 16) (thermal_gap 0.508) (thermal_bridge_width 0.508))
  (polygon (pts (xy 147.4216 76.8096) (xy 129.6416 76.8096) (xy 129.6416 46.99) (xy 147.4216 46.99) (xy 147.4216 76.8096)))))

